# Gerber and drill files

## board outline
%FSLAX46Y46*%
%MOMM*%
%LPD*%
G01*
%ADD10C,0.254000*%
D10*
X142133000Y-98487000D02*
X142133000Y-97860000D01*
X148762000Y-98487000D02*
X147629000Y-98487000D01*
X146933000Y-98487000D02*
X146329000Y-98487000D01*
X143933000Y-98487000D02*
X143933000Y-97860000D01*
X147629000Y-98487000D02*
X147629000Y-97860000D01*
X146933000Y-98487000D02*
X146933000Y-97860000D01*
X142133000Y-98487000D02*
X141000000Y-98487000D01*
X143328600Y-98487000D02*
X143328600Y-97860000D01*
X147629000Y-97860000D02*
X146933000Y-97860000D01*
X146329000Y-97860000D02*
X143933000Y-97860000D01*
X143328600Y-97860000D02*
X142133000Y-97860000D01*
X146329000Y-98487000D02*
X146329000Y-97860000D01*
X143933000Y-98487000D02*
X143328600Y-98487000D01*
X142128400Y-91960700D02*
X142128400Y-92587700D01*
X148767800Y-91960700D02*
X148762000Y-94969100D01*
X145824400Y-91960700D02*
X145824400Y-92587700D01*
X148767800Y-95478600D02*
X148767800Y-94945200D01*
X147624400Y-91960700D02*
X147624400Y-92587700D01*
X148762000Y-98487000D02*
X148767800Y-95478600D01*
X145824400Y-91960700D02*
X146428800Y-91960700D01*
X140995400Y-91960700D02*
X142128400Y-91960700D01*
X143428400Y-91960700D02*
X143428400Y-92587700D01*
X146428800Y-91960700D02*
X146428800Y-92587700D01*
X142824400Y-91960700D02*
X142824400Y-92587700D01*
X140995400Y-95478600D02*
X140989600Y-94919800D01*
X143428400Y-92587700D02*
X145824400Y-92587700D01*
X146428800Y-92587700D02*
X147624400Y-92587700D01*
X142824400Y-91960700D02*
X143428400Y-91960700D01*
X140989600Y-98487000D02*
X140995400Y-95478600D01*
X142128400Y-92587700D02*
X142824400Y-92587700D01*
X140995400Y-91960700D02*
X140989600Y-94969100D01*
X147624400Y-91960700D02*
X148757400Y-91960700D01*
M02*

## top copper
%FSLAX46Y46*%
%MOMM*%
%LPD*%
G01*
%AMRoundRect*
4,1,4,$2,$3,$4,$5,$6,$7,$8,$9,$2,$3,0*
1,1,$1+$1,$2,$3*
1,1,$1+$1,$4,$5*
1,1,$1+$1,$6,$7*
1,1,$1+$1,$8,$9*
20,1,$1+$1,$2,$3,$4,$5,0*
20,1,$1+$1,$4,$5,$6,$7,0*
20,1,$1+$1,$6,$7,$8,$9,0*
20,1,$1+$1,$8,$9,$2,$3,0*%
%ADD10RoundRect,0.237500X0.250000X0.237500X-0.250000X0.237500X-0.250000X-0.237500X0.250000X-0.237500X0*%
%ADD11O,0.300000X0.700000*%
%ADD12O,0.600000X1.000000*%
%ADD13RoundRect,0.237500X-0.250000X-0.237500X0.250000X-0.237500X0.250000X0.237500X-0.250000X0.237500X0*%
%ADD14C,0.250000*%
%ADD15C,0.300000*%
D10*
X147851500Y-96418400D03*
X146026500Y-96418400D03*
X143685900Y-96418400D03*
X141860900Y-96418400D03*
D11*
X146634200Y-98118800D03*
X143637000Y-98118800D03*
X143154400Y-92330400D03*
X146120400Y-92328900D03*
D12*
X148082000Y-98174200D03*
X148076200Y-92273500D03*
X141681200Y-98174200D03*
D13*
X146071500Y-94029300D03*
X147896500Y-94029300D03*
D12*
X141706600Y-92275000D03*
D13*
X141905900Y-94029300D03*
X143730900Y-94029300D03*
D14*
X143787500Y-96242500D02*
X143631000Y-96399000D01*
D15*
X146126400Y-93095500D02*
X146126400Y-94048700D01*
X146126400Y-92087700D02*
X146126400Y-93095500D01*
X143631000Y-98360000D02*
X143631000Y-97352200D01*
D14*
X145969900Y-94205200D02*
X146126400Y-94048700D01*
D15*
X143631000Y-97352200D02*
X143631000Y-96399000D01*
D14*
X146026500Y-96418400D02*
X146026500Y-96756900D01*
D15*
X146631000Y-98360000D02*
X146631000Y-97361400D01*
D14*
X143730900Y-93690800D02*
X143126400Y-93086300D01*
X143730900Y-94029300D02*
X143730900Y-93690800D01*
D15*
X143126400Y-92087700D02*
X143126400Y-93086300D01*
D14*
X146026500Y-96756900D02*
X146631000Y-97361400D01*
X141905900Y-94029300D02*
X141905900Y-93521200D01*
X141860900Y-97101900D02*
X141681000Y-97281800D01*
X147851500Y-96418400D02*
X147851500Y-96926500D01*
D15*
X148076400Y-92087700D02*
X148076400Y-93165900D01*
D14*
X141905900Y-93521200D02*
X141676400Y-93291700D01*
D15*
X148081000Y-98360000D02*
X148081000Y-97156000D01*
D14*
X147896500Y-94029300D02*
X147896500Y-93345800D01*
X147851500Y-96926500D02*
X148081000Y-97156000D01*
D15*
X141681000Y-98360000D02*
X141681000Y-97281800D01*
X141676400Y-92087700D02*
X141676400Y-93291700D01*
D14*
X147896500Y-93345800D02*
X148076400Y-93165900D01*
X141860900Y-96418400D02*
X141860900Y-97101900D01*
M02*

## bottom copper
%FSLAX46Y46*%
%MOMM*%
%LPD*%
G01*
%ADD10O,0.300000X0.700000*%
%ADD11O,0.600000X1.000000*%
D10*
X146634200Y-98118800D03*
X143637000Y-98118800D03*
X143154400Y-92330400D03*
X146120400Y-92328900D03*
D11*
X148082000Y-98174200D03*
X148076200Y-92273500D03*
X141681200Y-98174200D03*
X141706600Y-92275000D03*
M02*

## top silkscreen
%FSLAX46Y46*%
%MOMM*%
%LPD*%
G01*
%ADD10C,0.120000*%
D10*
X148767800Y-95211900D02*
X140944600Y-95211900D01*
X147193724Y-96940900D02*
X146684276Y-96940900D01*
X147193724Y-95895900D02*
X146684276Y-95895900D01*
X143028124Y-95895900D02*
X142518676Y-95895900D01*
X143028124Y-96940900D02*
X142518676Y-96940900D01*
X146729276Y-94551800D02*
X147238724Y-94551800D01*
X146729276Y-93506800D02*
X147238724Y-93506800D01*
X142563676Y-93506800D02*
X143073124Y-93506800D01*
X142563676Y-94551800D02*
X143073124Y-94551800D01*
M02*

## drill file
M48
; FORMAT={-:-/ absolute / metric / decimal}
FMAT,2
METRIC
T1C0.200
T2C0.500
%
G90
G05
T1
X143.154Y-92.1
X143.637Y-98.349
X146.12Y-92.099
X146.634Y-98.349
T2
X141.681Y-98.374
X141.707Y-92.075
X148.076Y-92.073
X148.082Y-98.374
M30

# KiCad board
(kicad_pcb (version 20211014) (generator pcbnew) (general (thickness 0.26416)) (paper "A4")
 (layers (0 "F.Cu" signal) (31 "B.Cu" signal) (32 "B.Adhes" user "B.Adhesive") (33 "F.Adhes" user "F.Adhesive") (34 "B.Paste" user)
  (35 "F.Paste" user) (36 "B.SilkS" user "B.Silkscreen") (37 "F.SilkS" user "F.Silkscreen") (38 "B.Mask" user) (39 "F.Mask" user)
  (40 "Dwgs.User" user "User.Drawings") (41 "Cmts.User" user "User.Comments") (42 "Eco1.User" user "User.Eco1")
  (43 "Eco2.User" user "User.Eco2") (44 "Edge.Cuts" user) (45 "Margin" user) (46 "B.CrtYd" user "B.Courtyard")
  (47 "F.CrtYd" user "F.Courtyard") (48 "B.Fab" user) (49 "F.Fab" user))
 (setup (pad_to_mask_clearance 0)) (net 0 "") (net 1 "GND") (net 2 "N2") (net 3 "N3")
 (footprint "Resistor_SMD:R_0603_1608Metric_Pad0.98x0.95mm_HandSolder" (layer "F.Cu") (at 146.939 96.4184 180)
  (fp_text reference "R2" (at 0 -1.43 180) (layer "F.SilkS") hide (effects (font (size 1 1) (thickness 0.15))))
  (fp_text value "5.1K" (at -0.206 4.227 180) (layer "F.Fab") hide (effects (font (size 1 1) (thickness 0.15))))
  (fp_line (start -0.254724 -0.5225) (end 0.254724 -0.5225) (layer "F.SilkS") (width 0.12))
  (fp_line (start -0.254724 0.5225) (end 0.254724 0.5225) (layer "F.SilkS") (width 0.12))
  (pad "1" smd roundrect (at -0.9125 0 180) (size 0.975 0.95) (layers "F.Cu" "F.Paste" "F.Mask") (roundrect_rratio 0.25) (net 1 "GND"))
  (pad "2" smd roundrect (at 0.9125 0 180) (size 0.975 0.95) (layers "F.Cu" "F.Paste" "F.Mask") (roundrect_rratio 0.25) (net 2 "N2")))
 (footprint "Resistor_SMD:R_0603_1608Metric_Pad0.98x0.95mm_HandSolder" (layer "F.Cu") (at 142.7734 96.4184 180)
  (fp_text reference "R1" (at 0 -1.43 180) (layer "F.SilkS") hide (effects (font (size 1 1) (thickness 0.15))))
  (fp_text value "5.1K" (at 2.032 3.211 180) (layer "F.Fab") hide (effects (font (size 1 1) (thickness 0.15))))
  (fp_line (start -0.254724 0.5225) (end 0.254724 0.5225) (layer "F.SilkS") (width 0.12))
  (fp_line (start -0.254724 -0.5225) (end 0.254724 -0.5225) (layer "F.SilkS") (width 0.12))
  (pad "1" smd roundrect (at -0.9125 0 180) (size 0.975 0.95) (layers "F.Cu" "F.Paste" "F.Mask") (roundrect_rratio 0.25) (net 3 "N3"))
  (pad "2" smd roundrect (at 0.9125 0 180) (size 0.975 0.95) (layers "F.Cu" "F.Paste" "F.Mask") (roundrect_rratio 0.25) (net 1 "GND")))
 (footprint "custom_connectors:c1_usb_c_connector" (layer "F.Cu") (at 151.7142 95.8088 90)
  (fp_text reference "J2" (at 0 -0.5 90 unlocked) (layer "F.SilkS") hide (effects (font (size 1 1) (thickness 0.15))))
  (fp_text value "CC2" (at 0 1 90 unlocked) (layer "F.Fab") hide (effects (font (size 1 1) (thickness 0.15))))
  (pad "1" thru_hole oval (at -2.54 -5.08 90) (size 0.7 0.3) (drill 0.2 (offset 0.23 0)) (layers *.Cu *.Mask) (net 2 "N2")))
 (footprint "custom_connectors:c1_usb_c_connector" (layer "F.Cu") (at 148.717 95.8088 90)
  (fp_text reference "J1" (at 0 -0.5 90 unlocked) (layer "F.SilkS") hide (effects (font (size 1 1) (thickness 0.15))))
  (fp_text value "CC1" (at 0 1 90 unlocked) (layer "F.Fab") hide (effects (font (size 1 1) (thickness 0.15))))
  (pad "1" thru_hole oval (at -2.54 -5.08 90) (size 0.7 0.3) (drill 0.2 (offset 0.23 0)) (layers *.Cu *.Mask) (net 3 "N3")))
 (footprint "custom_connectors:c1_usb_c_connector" (layer "F.Cu") (at 138.0744 94.6404 -90)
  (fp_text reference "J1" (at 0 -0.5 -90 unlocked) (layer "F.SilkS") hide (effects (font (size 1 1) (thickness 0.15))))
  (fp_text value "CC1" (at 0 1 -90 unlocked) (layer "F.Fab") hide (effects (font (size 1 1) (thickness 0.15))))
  (pad "1" thru_hole oval (at -2.54 -5.08 270) (size 0.7 0.3) (drill 0.2 (offset 0.23 0)) (layers F&B.Cu *.Mask)))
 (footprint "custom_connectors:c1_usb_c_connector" (layer "F.Cu") (at 141.0404 94.6389 -90)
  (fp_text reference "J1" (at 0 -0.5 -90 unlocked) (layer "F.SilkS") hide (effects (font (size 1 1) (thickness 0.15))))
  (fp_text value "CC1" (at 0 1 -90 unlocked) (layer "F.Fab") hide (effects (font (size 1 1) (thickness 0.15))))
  (pad "1" thru_hole oval (at -2.54 -5.08 270) (size 0.7 0.3) (drill 0.2 (offset 0.23 0)) (layers F&B.Cu *.Mask) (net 3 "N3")))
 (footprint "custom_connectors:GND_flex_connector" (layer "F.Cu") (at 153.162 98.3742 90)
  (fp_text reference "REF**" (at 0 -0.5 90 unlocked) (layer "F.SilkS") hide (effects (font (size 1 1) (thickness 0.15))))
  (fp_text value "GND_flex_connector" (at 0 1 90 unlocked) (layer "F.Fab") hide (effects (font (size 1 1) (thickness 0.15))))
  (pad "1" thru_hole oval (at 0 -5.08 90) (size 1 0.6) (drill 0.5 (offset 0.2 0)) (layers *.Cu *.Mask)))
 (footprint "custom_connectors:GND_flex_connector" (layer "F.Cu") (at 142.9962 92.0735 -90)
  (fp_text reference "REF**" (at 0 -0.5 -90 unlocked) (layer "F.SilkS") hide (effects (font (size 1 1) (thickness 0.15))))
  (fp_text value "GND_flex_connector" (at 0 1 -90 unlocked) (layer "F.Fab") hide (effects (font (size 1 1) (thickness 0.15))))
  (pad "1" thru_hole oval (at 0 -5.08 270) (size 1 0.6) (drill 0.5 (offset 0.2 0)) (layers F&B.Cu *.Mask)))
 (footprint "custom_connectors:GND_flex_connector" (layer "F.Cu") (at 146.7612 98.3742 90)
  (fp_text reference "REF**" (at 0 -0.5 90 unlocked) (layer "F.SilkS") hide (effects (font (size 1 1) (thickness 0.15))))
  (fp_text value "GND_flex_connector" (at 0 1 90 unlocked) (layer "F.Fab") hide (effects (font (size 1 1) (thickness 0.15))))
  (pad "1" thru_hole oval (at 0 -5.08 90) (size 1 0.6) (drill 0.5 (offset 0.2 0)) (layers *.Cu *.Mask)))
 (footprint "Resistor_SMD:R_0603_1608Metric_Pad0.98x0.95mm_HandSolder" (layer "F.Cu") (at 146.984 94.0293)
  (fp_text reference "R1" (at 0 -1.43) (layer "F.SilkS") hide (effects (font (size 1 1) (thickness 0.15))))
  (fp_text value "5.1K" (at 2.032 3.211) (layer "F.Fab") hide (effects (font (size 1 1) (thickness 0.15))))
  (fp_line (start -0.254724 0.5225) (end 0.254724 0.5225) (layer "F.SilkS") (width 0.12))
  (fp_line (start -0.254724 -0.5225) (end 0.254724 -0.5225) (layer "F.SilkS") (width 0.12))
  (pad "1" smd roundrect (at -0.9125 0) (size 0.975 0.95) (layers "F.Cu" "F.Paste" "F.Mask") (roundrect_rratio 0.25) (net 3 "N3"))
  (pad "2" smd roundrect (at 0.9125 0) (size 0.975 0.95) (layers "F.Cu" "F.Paste" "F.Mask") (roundrect_rratio 0.25) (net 1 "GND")))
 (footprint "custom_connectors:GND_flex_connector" (layer "F.Cu") (at 136.6266 92.075 -90)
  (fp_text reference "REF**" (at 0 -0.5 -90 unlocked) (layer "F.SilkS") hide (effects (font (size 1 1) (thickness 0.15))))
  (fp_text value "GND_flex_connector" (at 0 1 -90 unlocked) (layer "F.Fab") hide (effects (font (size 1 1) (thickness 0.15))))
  (pad "1" thru_hole oval (at 0 -5.08 270) (size 1 0.6) (drill 0.5 (offset 0.2 0)) (layers F&B.Cu *.Mask)))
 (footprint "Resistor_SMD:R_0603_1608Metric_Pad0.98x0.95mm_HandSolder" (layer "F.Cu") (at 142.8184 94.0293)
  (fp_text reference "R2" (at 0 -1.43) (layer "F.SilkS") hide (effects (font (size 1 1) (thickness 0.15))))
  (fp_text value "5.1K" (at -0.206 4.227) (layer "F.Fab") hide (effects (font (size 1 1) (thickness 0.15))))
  (fp_line (start -0.254724 -0.5225) (end 0.254724 -0.5225) (layer "F.SilkS") (width 0.12))
  (fp_line (start -0.254724 0.5225) (end 0.254724 0.5225) (layer "F.SilkS") (width 0.12))
  (pad "1" smd roundrect (at -0.9125 0) (size 0.975 0.95) (layers "F.Cu" "F.Paste" "F.Mask") (roundrect_rratio 0.25) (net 1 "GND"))
  (pad "2" smd roundrect (at 0.9125 0) (size 0.975 0.95) (layers "F.Cu" "F.Paste" "F.Mask") (roundrect_rratio 0.25) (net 2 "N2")))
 (gr_line (start 148.7678 95.2119) (end 140.9446 95.2119) (layer "F.SilkS") (width 0.12))
 (gr_line (start 142.133 98.487) (end 142.133 97.86) (layer "Edge.Cuts") (width 0.254))
 (gr_line (start 148.762 98.487) (end 147.629 98.487) (layer "Edge.Cuts") (width 0.254))
 (gr_line (start 146.933 98.487) (end 146.329 98.487) (layer "Edge.Cuts") (width 0.254))
 (gr_line (start 143.933 98.487) (end 143.933 97.86) (layer "Edge.Cuts") (width 0.254))
 (gr_line (start 147.629 98.487) (end 147.629 97.86) (layer "Edge.Cuts") (width 0.254))
 (gr_line (start 146.933 98.487) (end 146.933 97.86) (layer "Edge.Cuts") (width 0.254))
 (gr_line (start 142.133 98.487) (end 141 98.487) (layer "Edge.Cuts") (width 0.254))
 (gr_line (start 143.3286 98.487) (end 143.3286 97.86) (layer "Edge.Cuts") (width 0.254))
 (gr_line (start 147.629 97.86) (end 146.933 97.86) (layer "Edge.Cuts") (width 0.254))
 (gr_line (start 146.329 97.86) (end 143.933 97.86) (layer "Edge.Cuts") (width 0.254))
 (gr_line (start 143.3286 97.86) (end 142.133 97.86) (layer "Edge.Cuts") (width 0.254))
 (gr_line (start 146.329 98.487) (end 146.329 97.86) (layer "Edge.Cuts") (width 0.254))
 (gr_line (start 143.933 98.487) (end 143.3286 98.487) (layer "Edge.Cuts") (width 0.254))
 (gr_line (start 142.1284 91.9607) (end 142.1284 92.5877) (layer "Edge.Cuts") (width 0.254))
 (gr_line (start 148.7678 91.9607) (end 148.762 94.9691) (layer "Edge.Cuts") (width 0.254))
 (gr_line (start 145.8244 91.9607) (end 145.8244 92.5877) (layer "Edge.Cuts") (width 0.254))
 (gr_line (start 148.7678 95.4786) (end 148.7678 94.9452) (layer "Edge.Cuts") (width 0.254))
 (gr_line (start 147.6244 91.9607) (end 147.6244 92.5877) (layer "Edge.Cuts") (width 0.254))
 (gr_line (start 148.762 98.487) (end 148.7678 95.4786) (layer "Edge.Cuts") (width 0.254))
 (gr_line (start 145.8244 91.9607) (end 146.4288 91.9607) (layer "Edge.Cuts") (width 0.254))
 (gr_line (start 140.9954 91.9607) (end 142.1284 91.9607) (layer "Edge.Cuts") (width 0.254))
 (gr_line (start 143.4284 91.9607) (end 143.4284 92.5877) (layer "Edge.Cuts") (width 0.254))
 (gr_line (start 146.4288 91.9607) (end 146.4288 92.5877) (layer "Edge.Cuts") (width 0.254))
 (gr_line (start 142.8244 91.9607) (end 142.8244 92.5877) (layer "Edge.Cuts") (width 0.254))
 (gr_line (start 140.9954 95.4786) (end 140.9896 94.9198) (layer "Edge.Cuts") (width 0.254))
 (gr_line (start 143.4284 92.5877) (end 145.8244 92.5877) (layer "Edge.Cuts") (width 0.254))
 (gr_line (start 146.4288 92.5877) (end 147.6244 92.5877) (layer "Edge.Cuts") (width 0.254))
 (gr_line (start 142.8244 91.9607) (end 143.4284 91.9607) (layer "Edge.Cuts") (width 0.254))
 (gr_line (start 140.9896 98.487) (end 140.9954 95.4786) (layer "Edge.Cuts") (width 0.254))
 (gr_line (start 142.1284 92.5877) (end 142.8244 92.5877) (layer "Edge.Cuts") (width 0.254))
 (gr_line (start 140.9954 91.9607) (end 140.9896 94.9691) (layer "Edge.Cuts") (width 0.254))
 (gr_line (start 147.6244 91.9607) (end 148.7574 91.9607) (layer "Edge.Cuts") (width 0.254))
 (segment (start 143.7875 96.2425) (end 143.631 96.399) (width 0.25) (layer "F.Cu") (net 3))
 (segment (start 146.1264 93.0955) (end 146.1264 94.0487) (width 0.3) (layer "F.Cu") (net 3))
 (segment (start 146.1264 92.0877) (end 146.1264 93.0955) (width 0.3) (layer "F.Cu") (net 3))
 (segment (start 143.631 98.36) (end 143.631 97.3522) (width 0.3) (layer "F.Cu") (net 3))
 (segment (start 145.9699 94.2052) (end 146.1264 94.0487) (width 0.25) (layer "F.Cu") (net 3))
 (segment (start 143.631 97.3522) (end 143.631 96.399) (width 0.3) (layer "F.Cu") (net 3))
 (segment (start 146.0265 96.4184) (end 146.0265 96.7569) (width 0.25) (layer "F.Cu") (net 2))
 (segment (start 146.631 98.36) (end 146.631 97.3614) (width 0.3) (layer "F.Cu") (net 2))
 (segment (start 143.7309 93.6908) (end 143.1264 93.0863) (width 0.25) (layer "F.Cu") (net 2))
 (segment (start 143.7309 94.0293) (end 143.7309 93.6908) (width 0.25) (layer "F.Cu") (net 2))
 (segment (start 143.1264 92.0877) (end 143.1264 93.0863) (width 0.3) (layer "F.Cu") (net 2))
 (segment (start 146.0265 96.7569) (end 146.631 97.3614) (width 0.25) (layer "F.Cu") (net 2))
 (segment (start 141.9059 94.0293) (end 141.9059 93.5212) (width 0.25) (layer "F.Cu") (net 1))
 (segment (start 141.8609 97.1019) (end 141.681 97.2818) (width 0.25) (layer "F.Cu") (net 1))
 (segment (start 147.8515 96.4184) (end 147.8515 96.9265) (width 0.25) (layer "F.Cu") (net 1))
 (segment (start 148.0764 92.0877) (end 148.0764 93.1659) (width 0.3) (layer "F.Cu") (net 1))
 (segment (start 141.9059 93.5212) (end 141.6764 93.2917) (width 0.25) (layer "F.Cu") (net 1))
 (segment (start 148.081 98.36) (end 148.081 97.156) (width 0.3) (layer "F.Cu") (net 1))
 (segment (start 147.8965 94.0293) (end 147.8965 93.3458) (width 0.25) (layer "F.Cu") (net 1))
 (segment (start 147.8515 96.9265) (end 148.081 97.156) (width 0.25) (layer "F.Cu") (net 1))
 (segment (start 141.681 98.36) (end 141.681 97.2818) (width 0.3) (layer "F.Cu") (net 1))
 (segment (start 141.6764 92.0877) (end 141.6764 93.2917) (width 0.3) (layer "F.Cu") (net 1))
 (segment (start 147.8965 93.3458) (end 148.0764 93.1659) (width 0.25) (layer "F.Cu") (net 1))
 (segment (start 141.8609 96.4184) (end 141.8609 97.1019) (width 0.25) (layer "F.Cu") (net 1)))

